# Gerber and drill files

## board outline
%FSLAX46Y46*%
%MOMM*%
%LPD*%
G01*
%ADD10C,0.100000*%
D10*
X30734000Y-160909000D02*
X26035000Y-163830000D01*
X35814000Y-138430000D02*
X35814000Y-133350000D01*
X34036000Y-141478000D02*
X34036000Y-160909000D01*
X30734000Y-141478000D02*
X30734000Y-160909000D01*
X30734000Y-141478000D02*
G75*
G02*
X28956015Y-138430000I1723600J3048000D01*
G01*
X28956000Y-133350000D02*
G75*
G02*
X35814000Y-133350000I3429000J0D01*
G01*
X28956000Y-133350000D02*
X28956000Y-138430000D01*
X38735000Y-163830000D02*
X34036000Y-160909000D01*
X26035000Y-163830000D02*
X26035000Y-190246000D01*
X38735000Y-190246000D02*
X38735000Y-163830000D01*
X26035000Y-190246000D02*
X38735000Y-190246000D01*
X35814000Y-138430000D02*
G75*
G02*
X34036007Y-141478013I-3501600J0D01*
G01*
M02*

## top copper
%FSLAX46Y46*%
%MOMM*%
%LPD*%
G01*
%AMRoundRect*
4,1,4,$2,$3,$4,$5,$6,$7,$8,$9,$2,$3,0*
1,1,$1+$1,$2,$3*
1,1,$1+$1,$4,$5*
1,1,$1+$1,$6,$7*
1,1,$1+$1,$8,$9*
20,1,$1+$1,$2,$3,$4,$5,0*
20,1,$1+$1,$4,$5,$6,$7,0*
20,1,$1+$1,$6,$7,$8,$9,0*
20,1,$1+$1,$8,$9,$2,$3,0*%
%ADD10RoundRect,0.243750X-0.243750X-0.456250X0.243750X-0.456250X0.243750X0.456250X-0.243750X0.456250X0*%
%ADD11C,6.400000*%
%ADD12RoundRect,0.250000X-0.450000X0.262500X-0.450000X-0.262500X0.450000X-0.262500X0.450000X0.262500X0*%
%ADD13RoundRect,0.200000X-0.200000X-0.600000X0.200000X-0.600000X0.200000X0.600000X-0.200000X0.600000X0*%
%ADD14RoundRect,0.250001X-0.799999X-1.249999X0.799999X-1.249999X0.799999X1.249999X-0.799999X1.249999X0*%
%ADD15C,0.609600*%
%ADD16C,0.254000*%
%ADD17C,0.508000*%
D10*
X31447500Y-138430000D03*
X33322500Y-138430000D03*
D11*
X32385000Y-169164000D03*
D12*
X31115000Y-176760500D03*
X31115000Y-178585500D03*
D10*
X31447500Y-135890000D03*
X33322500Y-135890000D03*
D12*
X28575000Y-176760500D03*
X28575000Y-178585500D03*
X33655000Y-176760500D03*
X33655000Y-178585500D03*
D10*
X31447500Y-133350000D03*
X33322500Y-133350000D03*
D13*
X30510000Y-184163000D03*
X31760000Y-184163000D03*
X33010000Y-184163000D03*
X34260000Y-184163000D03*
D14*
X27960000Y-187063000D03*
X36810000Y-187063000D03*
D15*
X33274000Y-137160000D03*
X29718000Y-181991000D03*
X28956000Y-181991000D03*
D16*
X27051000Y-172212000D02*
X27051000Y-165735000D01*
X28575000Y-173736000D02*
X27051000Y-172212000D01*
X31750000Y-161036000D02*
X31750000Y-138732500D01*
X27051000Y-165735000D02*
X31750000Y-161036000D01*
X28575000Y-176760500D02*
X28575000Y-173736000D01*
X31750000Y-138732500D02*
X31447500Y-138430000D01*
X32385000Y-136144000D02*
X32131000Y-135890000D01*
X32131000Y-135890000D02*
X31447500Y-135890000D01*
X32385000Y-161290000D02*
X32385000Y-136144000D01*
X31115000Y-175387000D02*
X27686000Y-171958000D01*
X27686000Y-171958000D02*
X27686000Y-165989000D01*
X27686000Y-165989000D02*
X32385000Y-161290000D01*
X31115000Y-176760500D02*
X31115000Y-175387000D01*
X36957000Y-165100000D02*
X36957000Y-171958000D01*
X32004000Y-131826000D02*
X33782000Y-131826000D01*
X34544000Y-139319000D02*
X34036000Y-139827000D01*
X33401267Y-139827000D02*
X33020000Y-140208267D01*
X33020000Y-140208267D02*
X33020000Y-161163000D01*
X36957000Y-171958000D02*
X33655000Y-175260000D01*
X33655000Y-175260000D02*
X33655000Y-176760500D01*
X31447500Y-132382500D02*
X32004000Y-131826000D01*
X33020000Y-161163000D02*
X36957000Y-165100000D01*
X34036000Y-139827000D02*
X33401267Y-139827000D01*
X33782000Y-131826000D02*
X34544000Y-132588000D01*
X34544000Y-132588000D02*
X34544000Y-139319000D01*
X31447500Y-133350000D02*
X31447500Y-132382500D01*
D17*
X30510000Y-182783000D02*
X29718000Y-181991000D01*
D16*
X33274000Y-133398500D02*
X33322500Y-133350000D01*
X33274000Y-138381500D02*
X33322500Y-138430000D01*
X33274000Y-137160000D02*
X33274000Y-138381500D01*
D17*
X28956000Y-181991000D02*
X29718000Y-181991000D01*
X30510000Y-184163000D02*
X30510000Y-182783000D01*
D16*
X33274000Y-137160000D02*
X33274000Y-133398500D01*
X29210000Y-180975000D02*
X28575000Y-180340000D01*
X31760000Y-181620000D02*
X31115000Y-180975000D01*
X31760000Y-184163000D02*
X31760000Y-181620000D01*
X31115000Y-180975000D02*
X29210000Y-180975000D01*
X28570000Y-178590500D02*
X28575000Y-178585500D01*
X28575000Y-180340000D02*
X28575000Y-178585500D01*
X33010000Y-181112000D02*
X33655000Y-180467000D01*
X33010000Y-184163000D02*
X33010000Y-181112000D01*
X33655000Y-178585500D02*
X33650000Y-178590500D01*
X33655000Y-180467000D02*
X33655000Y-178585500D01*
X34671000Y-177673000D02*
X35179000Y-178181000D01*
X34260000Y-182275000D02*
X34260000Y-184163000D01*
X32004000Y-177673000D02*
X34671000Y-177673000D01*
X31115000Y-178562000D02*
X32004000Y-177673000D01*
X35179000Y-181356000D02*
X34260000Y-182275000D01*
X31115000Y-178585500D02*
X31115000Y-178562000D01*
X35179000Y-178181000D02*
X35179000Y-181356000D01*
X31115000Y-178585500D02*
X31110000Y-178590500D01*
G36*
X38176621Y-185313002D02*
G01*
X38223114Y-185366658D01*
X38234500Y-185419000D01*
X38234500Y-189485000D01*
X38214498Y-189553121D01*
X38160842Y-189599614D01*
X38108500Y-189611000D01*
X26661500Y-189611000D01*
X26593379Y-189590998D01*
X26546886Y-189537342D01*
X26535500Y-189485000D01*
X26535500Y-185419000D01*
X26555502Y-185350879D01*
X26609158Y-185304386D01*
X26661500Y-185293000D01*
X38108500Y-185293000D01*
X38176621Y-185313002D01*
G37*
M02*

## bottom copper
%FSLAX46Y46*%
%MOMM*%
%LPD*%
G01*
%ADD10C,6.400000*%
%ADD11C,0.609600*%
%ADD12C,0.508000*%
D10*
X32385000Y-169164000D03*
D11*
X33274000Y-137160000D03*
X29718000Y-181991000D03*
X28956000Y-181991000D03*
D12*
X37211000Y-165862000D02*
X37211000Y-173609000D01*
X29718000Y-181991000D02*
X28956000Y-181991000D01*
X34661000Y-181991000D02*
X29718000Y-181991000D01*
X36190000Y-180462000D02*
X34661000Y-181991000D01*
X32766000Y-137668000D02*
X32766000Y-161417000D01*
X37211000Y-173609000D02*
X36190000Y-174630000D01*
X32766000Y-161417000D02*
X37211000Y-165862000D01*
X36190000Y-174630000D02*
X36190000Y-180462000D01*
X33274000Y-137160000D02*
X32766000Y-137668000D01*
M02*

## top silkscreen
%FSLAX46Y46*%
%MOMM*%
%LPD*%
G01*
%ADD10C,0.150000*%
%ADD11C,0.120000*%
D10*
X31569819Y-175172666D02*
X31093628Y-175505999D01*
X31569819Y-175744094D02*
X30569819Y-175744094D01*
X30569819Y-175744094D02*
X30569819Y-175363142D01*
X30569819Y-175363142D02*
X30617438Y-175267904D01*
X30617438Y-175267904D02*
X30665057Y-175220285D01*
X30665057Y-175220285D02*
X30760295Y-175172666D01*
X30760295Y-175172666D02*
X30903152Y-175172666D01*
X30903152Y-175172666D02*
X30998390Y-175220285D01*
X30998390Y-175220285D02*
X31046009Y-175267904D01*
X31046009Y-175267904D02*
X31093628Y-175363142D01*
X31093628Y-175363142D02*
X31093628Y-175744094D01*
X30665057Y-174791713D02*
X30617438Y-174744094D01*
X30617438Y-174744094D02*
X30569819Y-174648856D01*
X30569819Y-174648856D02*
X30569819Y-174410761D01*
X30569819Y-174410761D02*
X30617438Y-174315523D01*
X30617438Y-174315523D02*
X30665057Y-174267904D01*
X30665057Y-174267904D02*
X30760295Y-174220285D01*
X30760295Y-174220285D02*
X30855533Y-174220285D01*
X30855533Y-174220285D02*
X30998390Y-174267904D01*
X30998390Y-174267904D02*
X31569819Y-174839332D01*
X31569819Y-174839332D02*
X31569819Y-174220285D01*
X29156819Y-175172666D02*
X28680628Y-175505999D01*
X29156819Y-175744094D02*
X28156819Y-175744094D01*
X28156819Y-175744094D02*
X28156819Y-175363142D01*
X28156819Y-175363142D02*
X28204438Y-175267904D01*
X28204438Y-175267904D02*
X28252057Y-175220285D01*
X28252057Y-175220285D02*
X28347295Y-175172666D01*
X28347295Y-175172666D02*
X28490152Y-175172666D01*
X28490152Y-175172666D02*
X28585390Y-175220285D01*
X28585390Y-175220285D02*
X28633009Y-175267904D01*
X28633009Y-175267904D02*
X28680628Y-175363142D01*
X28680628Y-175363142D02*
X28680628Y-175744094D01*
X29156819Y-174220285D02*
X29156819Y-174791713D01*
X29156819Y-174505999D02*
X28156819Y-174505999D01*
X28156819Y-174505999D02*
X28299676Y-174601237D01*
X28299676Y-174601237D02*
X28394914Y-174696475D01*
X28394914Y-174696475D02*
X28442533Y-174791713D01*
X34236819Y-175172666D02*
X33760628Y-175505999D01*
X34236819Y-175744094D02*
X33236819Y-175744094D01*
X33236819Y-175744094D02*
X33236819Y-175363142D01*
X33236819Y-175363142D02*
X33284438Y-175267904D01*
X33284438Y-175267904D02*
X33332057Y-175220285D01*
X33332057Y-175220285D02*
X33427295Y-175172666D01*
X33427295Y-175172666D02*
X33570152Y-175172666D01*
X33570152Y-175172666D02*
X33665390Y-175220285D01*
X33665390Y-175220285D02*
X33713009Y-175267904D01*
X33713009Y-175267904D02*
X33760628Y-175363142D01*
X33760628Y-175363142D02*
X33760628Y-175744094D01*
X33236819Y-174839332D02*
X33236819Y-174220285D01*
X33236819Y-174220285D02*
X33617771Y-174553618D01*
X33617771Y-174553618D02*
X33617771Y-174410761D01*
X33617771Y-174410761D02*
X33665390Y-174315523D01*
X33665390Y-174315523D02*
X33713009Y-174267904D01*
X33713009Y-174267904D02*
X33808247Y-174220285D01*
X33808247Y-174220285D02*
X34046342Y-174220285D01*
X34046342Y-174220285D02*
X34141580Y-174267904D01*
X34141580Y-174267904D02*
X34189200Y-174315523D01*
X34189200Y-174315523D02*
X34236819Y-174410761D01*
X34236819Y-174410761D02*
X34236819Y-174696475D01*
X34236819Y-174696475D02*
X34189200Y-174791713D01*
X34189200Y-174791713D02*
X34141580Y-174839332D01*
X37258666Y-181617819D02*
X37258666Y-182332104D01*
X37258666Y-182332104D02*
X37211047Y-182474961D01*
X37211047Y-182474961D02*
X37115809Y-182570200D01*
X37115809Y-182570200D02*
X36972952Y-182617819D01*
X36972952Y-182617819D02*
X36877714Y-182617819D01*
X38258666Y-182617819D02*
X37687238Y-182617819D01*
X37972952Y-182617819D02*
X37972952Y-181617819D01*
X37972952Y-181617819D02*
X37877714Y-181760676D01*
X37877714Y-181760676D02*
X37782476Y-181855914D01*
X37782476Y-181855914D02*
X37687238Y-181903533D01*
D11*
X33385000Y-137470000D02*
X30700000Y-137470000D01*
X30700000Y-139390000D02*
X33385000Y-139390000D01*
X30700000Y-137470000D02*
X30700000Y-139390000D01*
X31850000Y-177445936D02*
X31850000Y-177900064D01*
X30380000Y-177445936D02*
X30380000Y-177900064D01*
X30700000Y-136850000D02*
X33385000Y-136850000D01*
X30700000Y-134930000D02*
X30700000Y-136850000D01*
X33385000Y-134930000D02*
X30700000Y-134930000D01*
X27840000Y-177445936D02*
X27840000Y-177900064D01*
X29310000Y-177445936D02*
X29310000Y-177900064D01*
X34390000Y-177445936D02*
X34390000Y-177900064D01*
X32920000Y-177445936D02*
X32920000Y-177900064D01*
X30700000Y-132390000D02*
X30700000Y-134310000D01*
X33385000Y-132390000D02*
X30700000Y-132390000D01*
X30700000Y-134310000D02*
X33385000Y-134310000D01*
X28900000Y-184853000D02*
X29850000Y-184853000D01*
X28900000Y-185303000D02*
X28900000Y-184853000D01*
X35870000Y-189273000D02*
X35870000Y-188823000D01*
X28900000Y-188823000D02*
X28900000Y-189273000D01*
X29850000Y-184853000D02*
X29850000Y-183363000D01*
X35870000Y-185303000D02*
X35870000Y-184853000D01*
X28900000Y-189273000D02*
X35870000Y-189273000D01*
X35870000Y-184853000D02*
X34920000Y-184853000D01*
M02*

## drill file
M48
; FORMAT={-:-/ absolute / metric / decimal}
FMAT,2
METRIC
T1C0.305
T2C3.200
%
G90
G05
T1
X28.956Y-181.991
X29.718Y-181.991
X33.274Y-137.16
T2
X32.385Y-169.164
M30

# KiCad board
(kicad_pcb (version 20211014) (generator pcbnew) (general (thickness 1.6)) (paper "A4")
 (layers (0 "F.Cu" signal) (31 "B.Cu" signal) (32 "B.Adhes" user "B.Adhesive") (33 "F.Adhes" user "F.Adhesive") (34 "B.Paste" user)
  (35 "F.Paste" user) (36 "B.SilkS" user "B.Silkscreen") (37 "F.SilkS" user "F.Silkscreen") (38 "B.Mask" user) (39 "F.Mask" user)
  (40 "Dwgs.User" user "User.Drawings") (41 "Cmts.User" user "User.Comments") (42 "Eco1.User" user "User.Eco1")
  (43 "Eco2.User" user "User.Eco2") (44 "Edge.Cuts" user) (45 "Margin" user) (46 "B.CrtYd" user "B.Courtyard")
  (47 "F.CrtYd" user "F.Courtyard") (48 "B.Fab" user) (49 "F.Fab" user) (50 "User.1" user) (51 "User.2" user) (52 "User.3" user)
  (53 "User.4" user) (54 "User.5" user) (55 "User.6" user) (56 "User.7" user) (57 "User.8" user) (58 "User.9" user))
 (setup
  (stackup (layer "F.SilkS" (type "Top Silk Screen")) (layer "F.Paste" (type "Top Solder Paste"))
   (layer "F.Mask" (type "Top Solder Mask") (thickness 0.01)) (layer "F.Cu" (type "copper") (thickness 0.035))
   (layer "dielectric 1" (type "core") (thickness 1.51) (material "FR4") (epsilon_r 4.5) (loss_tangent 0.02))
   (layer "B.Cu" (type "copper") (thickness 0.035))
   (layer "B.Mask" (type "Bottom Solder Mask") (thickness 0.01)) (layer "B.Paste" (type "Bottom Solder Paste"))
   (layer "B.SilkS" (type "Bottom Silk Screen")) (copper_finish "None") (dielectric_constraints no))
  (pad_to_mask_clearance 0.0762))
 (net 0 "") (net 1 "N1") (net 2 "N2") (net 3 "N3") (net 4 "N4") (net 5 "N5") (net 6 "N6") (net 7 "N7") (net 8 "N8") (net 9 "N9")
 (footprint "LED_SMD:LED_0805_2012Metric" (layer "F.Cu") (at 32.385 138.43)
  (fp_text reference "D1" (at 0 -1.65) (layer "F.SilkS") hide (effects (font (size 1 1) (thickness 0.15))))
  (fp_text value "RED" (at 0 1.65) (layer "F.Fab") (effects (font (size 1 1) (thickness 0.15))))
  (fp_line (start 1 -0.96) (end -1.685 -0.96) (layer "F.SilkS") (width 0.12))
  (fp_line (start -1.685 0.96) (end 1 0.96) (layer "F.SilkS") (width 0.12))
  (fp_line (start -1.685 -0.96) (end -1.685 0.96) (layer "F.SilkS") (width 0.12))
  (pad "1" smd roundrect (at -0.9375 0) (size 0.975 1.4) (layers "F.Cu" "F.Paste" "F.Mask") (roundrect_rratio 0.25) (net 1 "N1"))
  (pad "2" smd roundrect (at 0.9375 0) (size 0.975 1.4) (layers "F.Cu" "F.Paste" "F.Mask") (roundrect_rratio 0.25) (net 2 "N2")))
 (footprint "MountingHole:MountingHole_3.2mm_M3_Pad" (layer "F.Cu") (at 32.385 169.164) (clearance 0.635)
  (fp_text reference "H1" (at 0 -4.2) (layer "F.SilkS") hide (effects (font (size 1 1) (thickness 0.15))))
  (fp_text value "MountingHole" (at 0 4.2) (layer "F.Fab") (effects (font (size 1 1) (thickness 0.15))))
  (pad "1" thru_hole circle (at 0 0) (size 6.4 6.4) (drill 3.2) (layers *.Cu *.Mask) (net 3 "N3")))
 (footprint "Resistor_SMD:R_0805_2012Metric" (layer "F.Cu") (at 31.115 177.673 -90)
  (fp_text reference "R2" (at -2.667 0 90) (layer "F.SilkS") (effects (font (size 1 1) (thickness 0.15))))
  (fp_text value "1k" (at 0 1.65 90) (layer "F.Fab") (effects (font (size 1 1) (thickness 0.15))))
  (fp_line (start -0.227064 -0.735) (end 0.227064 -0.735) (layer "F.SilkS") (width 0.12))
  (fp_line (start -0.227064 0.735) (end 0.227064 0.735) (layer "F.SilkS") (width 0.12))
  (pad "1" smd roundrect (at -0.9125 0 270) (size 1.025 1.4) (layers "F.Cu" "F.Paste" "F.Mask") (roundrect_rratio 0.243902) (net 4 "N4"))
  (pad "2" smd roundrect (at 0.9125 0 270) (size 1.025 1.4) (layers "F.Cu" "F.Paste" "F.Mask") (roundrect_rratio 0.243902) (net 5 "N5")))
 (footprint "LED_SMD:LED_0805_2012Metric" (layer "F.Cu") (at 32.385 135.89)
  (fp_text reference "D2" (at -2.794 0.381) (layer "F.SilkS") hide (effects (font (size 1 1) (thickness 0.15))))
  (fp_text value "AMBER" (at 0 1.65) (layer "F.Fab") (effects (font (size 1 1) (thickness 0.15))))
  (fp_line (start -1.685 0.96) (end 1 0.96) (layer "F.SilkS") (width 0.12))
  (fp_line (start -1.685 -0.96) (end -1.685 0.96) (layer "F.SilkS") (width 0.12))
  (fp_line (start 1 -0.96) (end -1.685 -0.96) (layer "F.SilkS") (width 0.12))
  (pad "1" smd roundrect (at -0.9375 0) (size 0.975 1.4) (layers "F.Cu" "F.Paste" "F.Mask") (roundrect_rratio 0.25) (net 4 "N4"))
  (pad "2" smd roundrect (at 0.9375 0) (size 0.975 1.4) (layers "F.Cu" "F.Paste" "F.Mask") (roundrect_rratio 0.25) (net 2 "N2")))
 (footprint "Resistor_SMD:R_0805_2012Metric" (layer "F.Cu") (at 28.575 177.673 -90)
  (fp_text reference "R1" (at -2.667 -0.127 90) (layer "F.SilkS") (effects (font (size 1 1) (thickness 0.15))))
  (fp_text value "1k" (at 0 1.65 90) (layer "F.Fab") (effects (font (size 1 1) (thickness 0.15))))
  (fp_line (start -0.227064 0.735) (end 0.227064 0.735) (layer "F.SilkS") (width 0.12))
  (fp_line (start -0.227064 -0.735) (end 0.227064 -0.735) (layer "F.SilkS") (width 0.12))
  (pad "1" smd roundrect (at -0.9125 0 270) (size 1.025 1.4) (layers "F.Cu" "F.Paste" "F.Mask") (roundrect_rratio 0.243902) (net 1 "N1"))
  (pad "2" smd roundrect (at 0.9125 0 270) (size 1.025 1.4) (layers "F.Cu" "F.Paste" "F.Mask") (roundrect_rratio 0.243902) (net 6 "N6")))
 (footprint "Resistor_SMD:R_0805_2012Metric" (layer "F.Cu") (at 33.655 177.673 -90)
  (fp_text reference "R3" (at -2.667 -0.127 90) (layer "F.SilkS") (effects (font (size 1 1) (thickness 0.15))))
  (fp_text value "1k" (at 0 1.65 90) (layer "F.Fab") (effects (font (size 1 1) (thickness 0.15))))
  (fp_line (start -0.227064 -0.735) (end 0.227064 -0.735) (layer "F.SilkS") (width 0.12))
  (fp_line (start -0.227064 0.735) (end 0.227064 0.735) (layer "F.SilkS") (width 0.12))
  (pad "1" smd roundrect (at -0.9125 0 270) (size 1.025 1.4) (layers "F.Cu" "F.Paste" "F.Mask") (roundrect_rratio 0.243902) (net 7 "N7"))
  (pad "2" smd roundrect (at 0.9125 0 270) (size 1.025 1.4) (layers "F.Cu" "F.Paste" "F.Mask") (roundrect_rratio 0.243902) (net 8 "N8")))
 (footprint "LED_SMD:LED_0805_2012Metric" (layer "F.Cu") (at 32.385 133.35)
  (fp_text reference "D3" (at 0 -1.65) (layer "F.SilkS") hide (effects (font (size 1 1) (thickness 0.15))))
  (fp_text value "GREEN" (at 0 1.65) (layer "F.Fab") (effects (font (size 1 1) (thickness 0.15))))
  (fp_line (start -1.685 -0.96) (end -1.685 0.96) (layer "F.SilkS") (width 0.12))
  (fp_line (start 1 -0.96) (end -1.685 -0.96) (layer "F.SilkS") (width 0.12))
  (fp_line (start -1.685 0.96) (end 1 0.96) (layer "F.SilkS") (width 0.12))
  (pad "1" smd roundrect (at -0.9375 0) (size 0.975 1.4) (layers "F.Cu" "F.Paste" "F.Mask") (roundrect_rratio 0.25) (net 7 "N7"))
  (pad "2" smd roundrect (at 0.9375 0) (size 0.975 1.4) (layers "F.Cu" "F.Paste" "F.Mask") (roundrect_rratio 0.25) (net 2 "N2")))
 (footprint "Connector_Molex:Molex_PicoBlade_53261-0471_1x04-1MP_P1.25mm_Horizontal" (layer "F.Cu") (at 32.385 186.563)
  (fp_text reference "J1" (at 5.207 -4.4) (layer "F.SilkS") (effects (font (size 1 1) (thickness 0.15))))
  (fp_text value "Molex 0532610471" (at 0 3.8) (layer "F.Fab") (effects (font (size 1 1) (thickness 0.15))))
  (fp_line (start -3.485 -1.71) (end -2.535 -1.71) (layer "F.SilkS") (width 0.12))
  (fp_line (start -3.485 -1.26) (end -3.485 -1.71) (layer "F.SilkS") (width 0.12))
  (fp_line (start 3.485 2.71) (end 3.485 2.26) (layer "F.SilkS") (width 0.12))
  (fp_line (start -3.485 2.26) (end -3.485 2.71) (layer "F.SilkS") (width 0.12))
  (fp_line (start -2.535 -1.71) (end -2.535 -3.2) (layer "F.SilkS") (width 0.12))
  (fp_line (start 3.485 -1.26) (end 3.485 -1.71) (layer "F.SilkS") (width 0.12))
  (fp_line (start -3.485 2.71) (end 3.485 2.71) (layer "F.SilkS") (width 0.12))
  (fp_line (start 3.485 -1.71) (end 2.535 -1.71) (layer "F.SilkS") (width 0.12))
  (pad "1" smd roundrect (at -1.875 -2.4) (size 0.8 1.6) (layers "F.Cu" "F.Paste" "F.Mask") (roundrect_rratio 0.25) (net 2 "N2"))
  (pad "2" smd roundrect (at -0.625 -2.4) (size 0.8 1.6) (layers "F.Cu" "F.Paste" "F.Mask") (roundrect_rratio 0.25) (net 6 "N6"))
  (pad "3" smd roundrect (at 0.625 -2.4) (size 0.8 1.6) (layers "F.Cu" "F.Paste" "F.Mask") (roundrect_rratio 0.25) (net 8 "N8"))
  (pad "4" smd roundrect (at 1.875 -2.4) (size 0.8 1.6) (layers "F.Cu" "F.Paste" "F.Mask") (roundrect_rratio 0.25) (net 5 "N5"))
  (pad "MP" smd roundrect (at -4.425 0.5) (size 2.1 3) (layers "F.Cu" "F.Paste" "F.Mask") (roundrect_rratio 0.119048) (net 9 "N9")
   (zone_connect 2))
  (pad "MP" smd roundrect (at 4.425 0.5) (size 2.1 3) (layers "F.Cu" "F.Paste" "F.Mask") (roundrect_rratio 0.119048) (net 9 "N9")
   (zone_connect 2)))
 (gr_line (start 30.734 160.909) (end 26.035 163.83) (layer "Edge.Cuts") (width 0.1))
 (gr_line (start 35.814 138.43) (end 35.814 133.35) (layer "Edge.Cuts") (width 0.1))
 (gr_line (start 34.036 141.478) (end 34.036 160.909) (layer "Edge.Cuts") (width 0.1))
 (gr_line (start 30.734 141.478) (end 30.734 160.909) (layer "Edge.Cuts") (width 0.1))
 (gr_arc (start 30.734 141.478) (mid 29.432988 140.19434) (end 28.956 138.43) (layer "Edge.Cuts") (width 0.1))
 (gr_arc (start 28.956 133.35) (mid 32.385 129.921) (end 35.814 133.35) (layer "Edge.Cuts") (width 0.1))
 (gr_line (start 28.956 133.35) (end 28.956 138.43) (layer "Edge.Cuts") (width 0.1))
 (gr_line (start 38.735 163.83) (end 34.036 160.909) (layer "Edge.Cuts") (width 0.1))
 (gr_line (start 26.035 163.83) (end 26.035 190.246) (layer "Edge.Cuts") (width 0.1))
 (gr_line (start 38.735 190.246) (end 38.735 163.83) (layer "Edge.Cuts") (width 0.1))
 (gr_line (start 26.035 190.246) (end 38.735 190.246) (layer "Edge.Cuts") (width 0.1))
 (gr_arc (start 35.814 138.43) (mid 35.337012 140.19434) (end 34.036 141.478) (layer "Edge.Cuts") (width 0.1))
 (segment (start 27.051 172.212) (end 27.051 165.735) (width 0.254) (layer "F.Cu") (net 1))
 (segment (start 28.575 173.736) (end 27.051 172.212) (width 0.254) (layer "F.Cu") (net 1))
 (segment (start 31.75 161.036) (end 31.75 138.7325) (width 0.254) (layer "F.Cu") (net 1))
 (segment (start 27.051 165.735) (end 31.75 161.036) (width 0.254) (layer "F.Cu") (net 1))
 (segment (start 28.575 176.7605) (end 28.575 173.736) (width 0.254) (layer "F.Cu") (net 1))
 (segment (start 31.75 138.7325) (end 31.4475 138.43) (width 0.254) (layer "F.Cu") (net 1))
 (segment (start 32.385 136.144) (end 32.131 135.89) (width 0.254) (layer "F.Cu") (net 4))
 (segment (start 32.131 135.89) (end 31.4475 135.89) (width 0.254) (layer "F.Cu") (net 4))
 (segment (start 32.385 161.29) (end 32.385 136.144) (width 0.254) (layer "F.Cu") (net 4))
 (segment (start 31.115 175.387) (end 27.686 171.958) (width 0.254) (layer "F.Cu") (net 4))
 (segment (start 27.686 171.958) (end 27.686 165.989) (width 0.254) (layer "F.Cu") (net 4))
 (segment (start 27.686 165.989) (end 32.385 161.29) (width 0.254) (layer "F.Cu") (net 4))
 (segment (start 31.115 176.7605) (end 31.115 175.387) (width 0.254) (layer "F.Cu") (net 4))
 (segment (start 36.957 165.1) (end 36.957 171.958) (width 0.254) (layer "F.Cu") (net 7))
 (segment (start 32.004 131.826) (end 33.782 131.826) (width 0.254) (layer "F.Cu") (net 7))
 (segment (start 34.544 139.319) (end 34.036 139.827) (width 0.254) (layer "F.Cu") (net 7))
 (segment (start 33.401267 139.827) (end 33.02 140.208267) (width 0.254) (layer "F.Cu") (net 7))
 (segment (start 33.02 140.208267) (end 33.02 161.163) (width 0.254) (layer "F.Cu") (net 7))
 (segment (start 36.957 171.958) (end 33.655 175.26) (width 0.254) (layer "F.Cu") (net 7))
 (segment (start 33.655 175.26) (end 33.655 176.7605) (width 0.254) (layer "F.Cu") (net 7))
 (segment (start 31.4475 132.3825) (end 32.004 131.826) (width 0.254) (layer "F.Cu") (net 7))
 (segment (start 33.02 161.163) (end 36.957 165.1) (width 0.254) (layer "F.Cu") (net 7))
 (segment (start 34.036 139.827) (end 33.401267 139.827) (width 0.254) (layer "F.Cu") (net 7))
 (segment (start 33.782 131.826) (end 34.544 132.588) (width 0.254) (layer "F.Cu") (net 7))
 (segment (start 34.544 132.588) (end 34.544 139.319) (width 0.254) (layer "F.Cu") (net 7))
 (segment (start 31.4475 133.35) (end 31.4475 132.3825) (width 0.254) (layer "F.Cu") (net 7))
 (segment (start 30.51 182.783) (end 29.718 181.991) (width 0.508) (layer "F.Cu") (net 2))
 (segment (start 33.274 133.3985) (end 33.3225 133.35) (width 0.254) (layer "F.Cu") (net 2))
 (segment (start 33.274 138.3815) (end 33.3225 138.43) (width 0.254) (layer "F.Cu") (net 2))
 (segment (start 33.274 137.16) (end 33.274 138.3815) (width 0.254) (layer "F.Cu") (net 2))
 (segment (start 28.956 181.991) (end 29.718 181.991) (width 0.508) (layer "F.Cu") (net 2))
 (segment (start 30.51 184.163) (end 30.51 182.783) (width 0.508) (layer "F.Cu") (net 2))
 (segment (start 33.274 137.16) (end 33.274 133.3985) (width 0.254) (layer "F.Cu") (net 2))
 (via (at 33.274 137.16) (size 0.6096) (drill 0.3048) (layers "F.Cu" "B.Cu") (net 2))
 (via (at 29.718 181.991) (size 0.6096) (drill 0.3048) (layers "F.Cu" "B.Cu") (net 2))
 (via (at 28.956 181.991) (size 0.6096) (drill 0.3048) (layers "F.Cu" "B.Cu") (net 2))
 (segment (start 37.211 165.862) (end 37.211 173.609) (width 0.508) (layer "B.Cu") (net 2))
 (segment (start 29.718 181.991) (end 28.956 181.991) (width 0.508) (layer "B.Cu") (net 2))
 (segment (start 34.661 181.991) (end 29.718 181.991) (width 0.508) (layer "B.Cu") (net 2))
 (segment (start 36.19 180.462) (end 34.661 181.991) (width 0.508) (layer "B.Cu") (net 2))
 (segment (start 32.766 137.668) (end 32.766 161.417) (width 0.508) (layer "B.Cu") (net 2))
 (segment (start 37.211 173.609) (end 36.19 174.63) (width 0.508) (layer "B.Cu") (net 2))
 (segment (start 32.766 161.417) (end 37.211 165.862) (width 0.508) (layer "B.Cu") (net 2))
 (segment (start 36.19 174.63) (end 36.19 180.462) (width 0.508) (layer "B.Cu") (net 2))
 (segment (start 33.274 137.16) (end 32.766 137.668) (width 0.508) (layer "B.Cu") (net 2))
 (segment (start 29.21 180.975) (end 28.575 180.34) (width 0.254) (layer "F.Cu") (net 6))
 (segment (start 31.76 181.62) (end 31.115 180.975) (width 0.254) (layer "F.Cu") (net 6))
 (segment (start 31.76 184.163) (end 31.76 181.62) (width 0.254) (layer "F.Cu") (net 6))
 (segment (start 31.115 180.975) (end 29.21 180.975) (width 0.254) (layer "F.Cu") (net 6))
 (segment (start 28.57 178.5905) (end 28.575 178.5855) (width 0.254) (layer "F.Cu") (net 6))
 (segment (start 28.575 180.34) (end 28.575 178.5855) (width 0.254) (layer "F.Cu") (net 6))
 (segment (start 33.01 181.112) (end 33.655 180.467) (width 0.254) (layer "F.Cu") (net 8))
 (segment (start 33.01 184.163) (end 33.01 181.112) (width 0.254) (layer "F.Cu") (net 8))
 (segment (start 33.655 178.5855) (end 33.65 178.5905) (width 0.254) (layer "F.Cu") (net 8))
 (segment (start 33.655 180.467) (end 33.655 178.5855) (width 0.254) (layer "F.Cu") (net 8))
 (segment (start 34.671 177.673) (end 35.179 178.181) (width 0.254) (layer "F.Cu") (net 5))
 (segment (start 34.26 182.275) (end 34.26 184.163) (width 0.254) (layer "F.Cu") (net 5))
 (segment (start 32.004 177.673) (end 34.671 177.673) (width 0.254) (layer "F.Cu") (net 5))
 (segment (start 31.115 178.562) (end 32.004 177.673) (width 0.254) (layer "F.Cu") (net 5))
 (segment (start 35.179 181.356) (end 34.26 182.275) (width 0.254) (layer "F.Cu") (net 5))
 (segment (start 31.115 178.5855) (end 31.115 178.562) (width 0.254) (layer "F.Cu") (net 5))
 (segment (start 35.179 178.181) (end 35.179 181.356) (width 0.254) (layer "F.Cu") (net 5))
 (segment (start 31.115 178.5855) (end 31.11 178.5905) (width 0.254) (layer "F.Cu") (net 5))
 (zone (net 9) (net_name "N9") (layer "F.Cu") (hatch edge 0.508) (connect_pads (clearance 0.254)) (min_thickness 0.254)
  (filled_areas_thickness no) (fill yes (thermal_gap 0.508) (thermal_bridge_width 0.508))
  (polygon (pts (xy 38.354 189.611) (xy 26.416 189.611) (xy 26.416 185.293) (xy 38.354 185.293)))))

